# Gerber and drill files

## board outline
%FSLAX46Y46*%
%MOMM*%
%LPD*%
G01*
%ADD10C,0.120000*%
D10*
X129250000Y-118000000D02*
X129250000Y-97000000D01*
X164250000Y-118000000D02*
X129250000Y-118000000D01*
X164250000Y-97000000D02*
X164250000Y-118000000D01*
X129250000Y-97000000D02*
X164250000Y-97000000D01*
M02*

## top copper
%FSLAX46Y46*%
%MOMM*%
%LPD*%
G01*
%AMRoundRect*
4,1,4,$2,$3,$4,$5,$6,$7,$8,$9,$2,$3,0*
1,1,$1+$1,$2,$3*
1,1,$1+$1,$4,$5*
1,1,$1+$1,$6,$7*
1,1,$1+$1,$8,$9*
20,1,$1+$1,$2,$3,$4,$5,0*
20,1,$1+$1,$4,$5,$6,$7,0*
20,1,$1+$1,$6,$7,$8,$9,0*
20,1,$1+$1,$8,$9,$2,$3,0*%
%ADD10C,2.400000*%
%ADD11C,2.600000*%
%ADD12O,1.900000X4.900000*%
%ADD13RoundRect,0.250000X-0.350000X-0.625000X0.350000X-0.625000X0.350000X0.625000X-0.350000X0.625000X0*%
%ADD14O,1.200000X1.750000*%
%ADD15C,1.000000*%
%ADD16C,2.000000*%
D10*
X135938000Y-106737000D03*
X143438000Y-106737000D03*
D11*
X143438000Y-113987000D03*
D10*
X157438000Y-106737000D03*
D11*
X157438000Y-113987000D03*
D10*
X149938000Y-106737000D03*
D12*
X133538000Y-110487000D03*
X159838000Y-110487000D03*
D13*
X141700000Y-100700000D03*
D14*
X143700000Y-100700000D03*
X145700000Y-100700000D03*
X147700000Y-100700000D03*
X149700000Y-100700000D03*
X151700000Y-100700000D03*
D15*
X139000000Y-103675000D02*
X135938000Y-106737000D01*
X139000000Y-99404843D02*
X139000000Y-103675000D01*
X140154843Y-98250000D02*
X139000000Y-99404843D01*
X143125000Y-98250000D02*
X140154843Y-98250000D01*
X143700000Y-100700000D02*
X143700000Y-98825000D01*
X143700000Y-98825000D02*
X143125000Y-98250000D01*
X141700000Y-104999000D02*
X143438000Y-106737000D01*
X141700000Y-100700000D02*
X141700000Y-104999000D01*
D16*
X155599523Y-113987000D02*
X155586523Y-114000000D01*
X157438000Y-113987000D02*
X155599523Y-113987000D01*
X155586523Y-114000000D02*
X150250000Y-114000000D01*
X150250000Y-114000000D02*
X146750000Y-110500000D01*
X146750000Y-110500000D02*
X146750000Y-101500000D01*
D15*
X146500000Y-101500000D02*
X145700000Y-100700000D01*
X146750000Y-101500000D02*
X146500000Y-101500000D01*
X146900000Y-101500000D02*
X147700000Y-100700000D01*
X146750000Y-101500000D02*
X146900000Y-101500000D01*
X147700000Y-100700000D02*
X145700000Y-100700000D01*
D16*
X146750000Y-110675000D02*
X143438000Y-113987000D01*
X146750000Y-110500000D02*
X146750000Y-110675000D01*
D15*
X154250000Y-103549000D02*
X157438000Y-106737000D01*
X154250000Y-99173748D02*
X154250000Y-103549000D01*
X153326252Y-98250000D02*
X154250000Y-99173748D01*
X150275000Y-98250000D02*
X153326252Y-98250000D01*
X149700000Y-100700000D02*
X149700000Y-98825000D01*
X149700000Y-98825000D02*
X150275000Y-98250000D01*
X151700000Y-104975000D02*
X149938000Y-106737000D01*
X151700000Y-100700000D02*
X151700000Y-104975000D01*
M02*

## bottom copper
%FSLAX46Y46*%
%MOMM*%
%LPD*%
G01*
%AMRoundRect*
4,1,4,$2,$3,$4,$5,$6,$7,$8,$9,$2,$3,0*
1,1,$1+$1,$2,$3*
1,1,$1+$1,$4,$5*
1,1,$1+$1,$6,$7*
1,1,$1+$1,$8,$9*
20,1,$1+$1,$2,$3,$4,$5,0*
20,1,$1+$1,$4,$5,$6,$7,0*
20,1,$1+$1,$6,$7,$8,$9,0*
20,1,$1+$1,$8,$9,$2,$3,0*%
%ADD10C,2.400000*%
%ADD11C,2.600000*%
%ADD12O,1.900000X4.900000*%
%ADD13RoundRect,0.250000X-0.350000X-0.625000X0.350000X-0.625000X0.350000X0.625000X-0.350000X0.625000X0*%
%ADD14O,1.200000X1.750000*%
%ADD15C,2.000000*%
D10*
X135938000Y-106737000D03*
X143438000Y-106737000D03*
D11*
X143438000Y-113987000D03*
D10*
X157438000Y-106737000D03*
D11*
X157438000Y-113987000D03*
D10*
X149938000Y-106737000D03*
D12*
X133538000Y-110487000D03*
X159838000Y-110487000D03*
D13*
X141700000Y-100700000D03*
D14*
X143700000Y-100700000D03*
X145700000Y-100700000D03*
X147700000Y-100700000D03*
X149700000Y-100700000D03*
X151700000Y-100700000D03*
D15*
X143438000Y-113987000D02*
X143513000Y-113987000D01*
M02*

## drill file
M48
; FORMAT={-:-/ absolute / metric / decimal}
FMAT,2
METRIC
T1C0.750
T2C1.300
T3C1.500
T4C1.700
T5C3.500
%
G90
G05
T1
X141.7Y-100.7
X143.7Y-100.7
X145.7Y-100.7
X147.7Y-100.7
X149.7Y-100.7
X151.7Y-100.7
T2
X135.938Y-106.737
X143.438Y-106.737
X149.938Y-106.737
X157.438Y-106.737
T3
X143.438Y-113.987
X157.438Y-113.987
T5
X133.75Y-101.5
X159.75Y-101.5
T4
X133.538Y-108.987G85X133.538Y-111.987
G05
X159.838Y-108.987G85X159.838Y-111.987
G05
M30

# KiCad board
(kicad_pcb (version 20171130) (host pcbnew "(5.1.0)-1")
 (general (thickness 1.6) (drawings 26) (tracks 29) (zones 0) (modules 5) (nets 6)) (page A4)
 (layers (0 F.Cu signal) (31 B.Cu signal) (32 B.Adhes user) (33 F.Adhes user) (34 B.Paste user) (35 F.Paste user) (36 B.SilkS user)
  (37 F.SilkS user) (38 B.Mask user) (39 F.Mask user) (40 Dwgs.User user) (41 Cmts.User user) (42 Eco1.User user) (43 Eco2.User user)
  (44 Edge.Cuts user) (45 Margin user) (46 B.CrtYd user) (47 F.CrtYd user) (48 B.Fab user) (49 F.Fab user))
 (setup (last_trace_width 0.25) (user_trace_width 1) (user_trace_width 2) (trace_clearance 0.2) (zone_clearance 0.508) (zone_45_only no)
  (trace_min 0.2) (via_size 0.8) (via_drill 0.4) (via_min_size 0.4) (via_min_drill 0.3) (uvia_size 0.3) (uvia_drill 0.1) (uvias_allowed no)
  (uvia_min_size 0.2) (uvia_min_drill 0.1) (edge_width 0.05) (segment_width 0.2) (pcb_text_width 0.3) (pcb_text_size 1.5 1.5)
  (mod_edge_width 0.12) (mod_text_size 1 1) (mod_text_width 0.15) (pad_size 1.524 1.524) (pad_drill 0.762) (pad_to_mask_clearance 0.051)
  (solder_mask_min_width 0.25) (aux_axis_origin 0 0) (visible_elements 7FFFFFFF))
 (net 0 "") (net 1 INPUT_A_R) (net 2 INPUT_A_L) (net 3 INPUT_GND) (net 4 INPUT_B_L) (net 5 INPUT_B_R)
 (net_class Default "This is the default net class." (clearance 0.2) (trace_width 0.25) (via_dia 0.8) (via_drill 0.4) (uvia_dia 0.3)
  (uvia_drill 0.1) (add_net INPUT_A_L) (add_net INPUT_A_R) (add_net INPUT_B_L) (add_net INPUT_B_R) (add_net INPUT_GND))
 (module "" (layer F.Cu) (at 140.5 94.25)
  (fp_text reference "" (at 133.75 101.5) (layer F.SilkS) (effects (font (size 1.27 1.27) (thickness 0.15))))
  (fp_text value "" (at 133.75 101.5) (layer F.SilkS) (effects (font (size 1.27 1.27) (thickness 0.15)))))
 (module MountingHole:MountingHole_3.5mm (layer F.Cu) (at 133.75 101.5)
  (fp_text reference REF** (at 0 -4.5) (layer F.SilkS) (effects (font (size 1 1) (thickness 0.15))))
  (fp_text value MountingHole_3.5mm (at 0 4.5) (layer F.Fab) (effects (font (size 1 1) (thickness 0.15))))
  (pad 1 np_thru_hole circle (at 0 0) (size 3.5 3.5) (drill 3.5) (layers *.Cu *.Mask)))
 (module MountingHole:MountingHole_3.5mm (layer F.Cu) (at 159.75 101.5)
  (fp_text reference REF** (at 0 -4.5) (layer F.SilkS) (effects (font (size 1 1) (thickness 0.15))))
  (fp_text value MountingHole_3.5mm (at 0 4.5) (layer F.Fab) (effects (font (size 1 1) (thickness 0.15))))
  (pad 1 np_thru_hole circle (at 0 0) (size 3.5 3.5) (drill 3.5) (layers *.Cu *.Mask)))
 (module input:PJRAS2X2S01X (layer F.Cu) (at 135.938 106.737)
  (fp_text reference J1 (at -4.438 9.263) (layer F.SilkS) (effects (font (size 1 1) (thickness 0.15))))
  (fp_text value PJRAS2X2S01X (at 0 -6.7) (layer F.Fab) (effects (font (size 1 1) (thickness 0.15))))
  (pad 1 thru_hole circle (at 0 0) (size 2.4 2.4) (drill 1.3) (layers *.Cu *.Mask) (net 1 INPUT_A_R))
  (pad 3 thru_hole circle (at 7.5 0) (size 2.4 2.4) (drill 1.3) (layers *.Cu *.Mask) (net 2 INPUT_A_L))
  (pad 2 thru_hole circle (at 7.5 7.25) (size 2.6 2.6) (drill 1.5) (layers *.Cu *.Mask) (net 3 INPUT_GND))
  (pad 6 thru_hole circle (at 21.5 0) (size 2.4 2.4) (drill 1.3) (layers *.Cu *.Mask) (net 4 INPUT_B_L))
  (pad 5 thru_hole circle (at 21.5 7.25) (size 2.6 2.6) (drill 1.5) (layers *.Cu *.Mask) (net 3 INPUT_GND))
  (pad 4 thru_hole circle (at 14 0) (size 2.4 2.4) (drill 1.3) (layers *.Cu *.Mask) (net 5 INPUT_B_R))
  (pad 0 thru_hole oval (at -2.4 3.75) (size 1.9 4.9) (drill oval 1.7 4.7) (layers *.Cu *.Mask))
  (pad 0 thru_hole oval (at 23.9 3.75) (size 1.9 4.9) (drill oval 1.7 4.7) (layers *.Cu *.Mask)))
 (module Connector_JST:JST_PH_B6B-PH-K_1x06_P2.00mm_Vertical (layer F.Cu) (at 141.7 100.7)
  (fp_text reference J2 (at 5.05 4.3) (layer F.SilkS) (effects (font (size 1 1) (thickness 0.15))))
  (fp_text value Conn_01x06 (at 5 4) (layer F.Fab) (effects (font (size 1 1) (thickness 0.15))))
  (pad 1 thru_hole roundrect (at 0 0) (size 1.2 1.75) (drill 0.75) (layers *.Cu *.Mask) (roundrect_rratio 0.208333) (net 2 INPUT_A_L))
  (pad 2 thru_hole oval (at 2 0) (size 1.2 1.75) (drill 0.75) (layers *.Cu *.Mask) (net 1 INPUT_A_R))
  (pad 3 thru_hole oval (at 4 0) (size 1.2 1.75) (drill 0.75) (layers *.Cu *.Mask) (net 3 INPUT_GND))
  (pad 4 thru_hole oval (at 6 0) (size 1.2 1.75) (drill 0.75) (layers *.Cu *.Mask) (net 3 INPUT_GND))
  (pad 5 thru_hole oval (at 8 0) (size 1.2 1.75) (drill 0.75) (layers *.Cu *.Mask) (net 4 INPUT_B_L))
  (pad 6 thru_hole oval (at 10 0) (size 1.2 1.75) (drill 0.75) (layers *.Cu *.Mask) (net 5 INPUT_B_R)))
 (gr_line (start 129.25 118) (end 129.25 97) (layer Edge.Cuts) (width 0.12))
 (gr_line (start 164.25 118) (end 129.25 118) (layer Edge.Cuts) (width 0.12))
 (gr_line (start 164.25 97) (end 164.25 118) (layer Edge.Cuts) (width 0.12))
 (gr_line (start 129.25 97) (end 164.25 97) (layer Edge.Cuts) (width 0.12))
 (segment (start 139 103.675) (end 135.938 106.737) (width 1) (layer F.Cu) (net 1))
 (segment (start 139 99.404843) (end 139 103.675) (width 1) (layer F.Cu) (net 1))
 (segment (start 140.154843 98.25) (end 139 99.404843) (width 1) (layer F.Cu) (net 1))
 (segment (start 143.125 98.25) (end 140.154843 98.25) (width 1) (layer F.Cu) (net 1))
 (segment (start 143.7 100.7) (end 143.7 98.825) (width 1) (layer F.Cu) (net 1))
 (segment (start 143.7 98.825) (end 143.125 98.25) (width 1) (layer F.Cu) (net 1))
 (segment (start 141.7 104.999) (end 143.438 106.737) (width 1) (layer F.Cu) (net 2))
 (segment (start 141.7 100.7) (end 141.7 104.999) (width 1) (layer F.Cu) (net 2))
 (segment (start 155.599523 113.987) (end 155.586523 114) (width 2) (layer F.Cu) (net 3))
 (segment (start 157.438 113.987) (end 155.599523 113.987) (width 2) (layer F.Cu) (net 3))
 (segment (start 155.586523 114) (end 150.25 114) (width 2) (layer F.Cu) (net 3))
 (segment (start 150.25 114) (end 146.75 110.5) (width 2) (layer F.Cu) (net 3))
 (segment (start 146.75 110.5) (end 146.75 101.5) (width 2) (layer F.Cu) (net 3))
 (segment (start 146.5 101.5) (end 145.7 100.7) (width 1) (layer F.Cu) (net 3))
 (segment (start 146.75 101.5) (end 146.5 101.5) (width 1) (layer F.Cu) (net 3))
 (segment (start 146.9 101.5) (end 147.7 100.7) (width 1) (layer F.Cu) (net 3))
 (segment (start 146.75 101.5) (end 146.9 101.5) (width 1) (layer F.Cu) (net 3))
 (segment (start 143.438 113.987) (end 143.513 113.987) (width 2) (layer B.Cu) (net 3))
 (segment (start 147.7 100.7) (end 145.7 100.7) (width 1) (layer F.Cu) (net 3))
 (segment (start 146.75 110.675) (end 143.438 113.987) (width 2) (layer F.Cu) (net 3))
 (segment (start 146.75 110.5) (end 146.75 110.675) (width 2) (layer F.Cu) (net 3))
 (segment (start 154.25 103.549) (end 157.438 106.737) (width 1) (layer F.Cu) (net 4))
 (segment (start 154.25 99.173748) (end 154.25 103.549) (width 1) (layer F.Cu) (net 4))
 (segment (start 153.326252 98.25) (end 154.25 99.173748) (width 1) (layer F.Cu) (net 4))
 (segment (start 150.275 98.25) (end 153.326252 98.25) (width 1) (layer F.Cu) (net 4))
 (segment (start 149.7 100.7) (end 149.7 98.825) (width 1) (layer F.Cu) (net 4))
 (segment (start 149.7 98.825) (end 150.275 98.25) (width 1) (layer F.Cu) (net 4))
 (segment (start 151.7 104.975) (end 149.938 106.737) (width 1) (layer F.Cu) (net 5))
 (segment (start 151.7 100.7) (end 151.7 104.975) (width 1) (layer F.Cu) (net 5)))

